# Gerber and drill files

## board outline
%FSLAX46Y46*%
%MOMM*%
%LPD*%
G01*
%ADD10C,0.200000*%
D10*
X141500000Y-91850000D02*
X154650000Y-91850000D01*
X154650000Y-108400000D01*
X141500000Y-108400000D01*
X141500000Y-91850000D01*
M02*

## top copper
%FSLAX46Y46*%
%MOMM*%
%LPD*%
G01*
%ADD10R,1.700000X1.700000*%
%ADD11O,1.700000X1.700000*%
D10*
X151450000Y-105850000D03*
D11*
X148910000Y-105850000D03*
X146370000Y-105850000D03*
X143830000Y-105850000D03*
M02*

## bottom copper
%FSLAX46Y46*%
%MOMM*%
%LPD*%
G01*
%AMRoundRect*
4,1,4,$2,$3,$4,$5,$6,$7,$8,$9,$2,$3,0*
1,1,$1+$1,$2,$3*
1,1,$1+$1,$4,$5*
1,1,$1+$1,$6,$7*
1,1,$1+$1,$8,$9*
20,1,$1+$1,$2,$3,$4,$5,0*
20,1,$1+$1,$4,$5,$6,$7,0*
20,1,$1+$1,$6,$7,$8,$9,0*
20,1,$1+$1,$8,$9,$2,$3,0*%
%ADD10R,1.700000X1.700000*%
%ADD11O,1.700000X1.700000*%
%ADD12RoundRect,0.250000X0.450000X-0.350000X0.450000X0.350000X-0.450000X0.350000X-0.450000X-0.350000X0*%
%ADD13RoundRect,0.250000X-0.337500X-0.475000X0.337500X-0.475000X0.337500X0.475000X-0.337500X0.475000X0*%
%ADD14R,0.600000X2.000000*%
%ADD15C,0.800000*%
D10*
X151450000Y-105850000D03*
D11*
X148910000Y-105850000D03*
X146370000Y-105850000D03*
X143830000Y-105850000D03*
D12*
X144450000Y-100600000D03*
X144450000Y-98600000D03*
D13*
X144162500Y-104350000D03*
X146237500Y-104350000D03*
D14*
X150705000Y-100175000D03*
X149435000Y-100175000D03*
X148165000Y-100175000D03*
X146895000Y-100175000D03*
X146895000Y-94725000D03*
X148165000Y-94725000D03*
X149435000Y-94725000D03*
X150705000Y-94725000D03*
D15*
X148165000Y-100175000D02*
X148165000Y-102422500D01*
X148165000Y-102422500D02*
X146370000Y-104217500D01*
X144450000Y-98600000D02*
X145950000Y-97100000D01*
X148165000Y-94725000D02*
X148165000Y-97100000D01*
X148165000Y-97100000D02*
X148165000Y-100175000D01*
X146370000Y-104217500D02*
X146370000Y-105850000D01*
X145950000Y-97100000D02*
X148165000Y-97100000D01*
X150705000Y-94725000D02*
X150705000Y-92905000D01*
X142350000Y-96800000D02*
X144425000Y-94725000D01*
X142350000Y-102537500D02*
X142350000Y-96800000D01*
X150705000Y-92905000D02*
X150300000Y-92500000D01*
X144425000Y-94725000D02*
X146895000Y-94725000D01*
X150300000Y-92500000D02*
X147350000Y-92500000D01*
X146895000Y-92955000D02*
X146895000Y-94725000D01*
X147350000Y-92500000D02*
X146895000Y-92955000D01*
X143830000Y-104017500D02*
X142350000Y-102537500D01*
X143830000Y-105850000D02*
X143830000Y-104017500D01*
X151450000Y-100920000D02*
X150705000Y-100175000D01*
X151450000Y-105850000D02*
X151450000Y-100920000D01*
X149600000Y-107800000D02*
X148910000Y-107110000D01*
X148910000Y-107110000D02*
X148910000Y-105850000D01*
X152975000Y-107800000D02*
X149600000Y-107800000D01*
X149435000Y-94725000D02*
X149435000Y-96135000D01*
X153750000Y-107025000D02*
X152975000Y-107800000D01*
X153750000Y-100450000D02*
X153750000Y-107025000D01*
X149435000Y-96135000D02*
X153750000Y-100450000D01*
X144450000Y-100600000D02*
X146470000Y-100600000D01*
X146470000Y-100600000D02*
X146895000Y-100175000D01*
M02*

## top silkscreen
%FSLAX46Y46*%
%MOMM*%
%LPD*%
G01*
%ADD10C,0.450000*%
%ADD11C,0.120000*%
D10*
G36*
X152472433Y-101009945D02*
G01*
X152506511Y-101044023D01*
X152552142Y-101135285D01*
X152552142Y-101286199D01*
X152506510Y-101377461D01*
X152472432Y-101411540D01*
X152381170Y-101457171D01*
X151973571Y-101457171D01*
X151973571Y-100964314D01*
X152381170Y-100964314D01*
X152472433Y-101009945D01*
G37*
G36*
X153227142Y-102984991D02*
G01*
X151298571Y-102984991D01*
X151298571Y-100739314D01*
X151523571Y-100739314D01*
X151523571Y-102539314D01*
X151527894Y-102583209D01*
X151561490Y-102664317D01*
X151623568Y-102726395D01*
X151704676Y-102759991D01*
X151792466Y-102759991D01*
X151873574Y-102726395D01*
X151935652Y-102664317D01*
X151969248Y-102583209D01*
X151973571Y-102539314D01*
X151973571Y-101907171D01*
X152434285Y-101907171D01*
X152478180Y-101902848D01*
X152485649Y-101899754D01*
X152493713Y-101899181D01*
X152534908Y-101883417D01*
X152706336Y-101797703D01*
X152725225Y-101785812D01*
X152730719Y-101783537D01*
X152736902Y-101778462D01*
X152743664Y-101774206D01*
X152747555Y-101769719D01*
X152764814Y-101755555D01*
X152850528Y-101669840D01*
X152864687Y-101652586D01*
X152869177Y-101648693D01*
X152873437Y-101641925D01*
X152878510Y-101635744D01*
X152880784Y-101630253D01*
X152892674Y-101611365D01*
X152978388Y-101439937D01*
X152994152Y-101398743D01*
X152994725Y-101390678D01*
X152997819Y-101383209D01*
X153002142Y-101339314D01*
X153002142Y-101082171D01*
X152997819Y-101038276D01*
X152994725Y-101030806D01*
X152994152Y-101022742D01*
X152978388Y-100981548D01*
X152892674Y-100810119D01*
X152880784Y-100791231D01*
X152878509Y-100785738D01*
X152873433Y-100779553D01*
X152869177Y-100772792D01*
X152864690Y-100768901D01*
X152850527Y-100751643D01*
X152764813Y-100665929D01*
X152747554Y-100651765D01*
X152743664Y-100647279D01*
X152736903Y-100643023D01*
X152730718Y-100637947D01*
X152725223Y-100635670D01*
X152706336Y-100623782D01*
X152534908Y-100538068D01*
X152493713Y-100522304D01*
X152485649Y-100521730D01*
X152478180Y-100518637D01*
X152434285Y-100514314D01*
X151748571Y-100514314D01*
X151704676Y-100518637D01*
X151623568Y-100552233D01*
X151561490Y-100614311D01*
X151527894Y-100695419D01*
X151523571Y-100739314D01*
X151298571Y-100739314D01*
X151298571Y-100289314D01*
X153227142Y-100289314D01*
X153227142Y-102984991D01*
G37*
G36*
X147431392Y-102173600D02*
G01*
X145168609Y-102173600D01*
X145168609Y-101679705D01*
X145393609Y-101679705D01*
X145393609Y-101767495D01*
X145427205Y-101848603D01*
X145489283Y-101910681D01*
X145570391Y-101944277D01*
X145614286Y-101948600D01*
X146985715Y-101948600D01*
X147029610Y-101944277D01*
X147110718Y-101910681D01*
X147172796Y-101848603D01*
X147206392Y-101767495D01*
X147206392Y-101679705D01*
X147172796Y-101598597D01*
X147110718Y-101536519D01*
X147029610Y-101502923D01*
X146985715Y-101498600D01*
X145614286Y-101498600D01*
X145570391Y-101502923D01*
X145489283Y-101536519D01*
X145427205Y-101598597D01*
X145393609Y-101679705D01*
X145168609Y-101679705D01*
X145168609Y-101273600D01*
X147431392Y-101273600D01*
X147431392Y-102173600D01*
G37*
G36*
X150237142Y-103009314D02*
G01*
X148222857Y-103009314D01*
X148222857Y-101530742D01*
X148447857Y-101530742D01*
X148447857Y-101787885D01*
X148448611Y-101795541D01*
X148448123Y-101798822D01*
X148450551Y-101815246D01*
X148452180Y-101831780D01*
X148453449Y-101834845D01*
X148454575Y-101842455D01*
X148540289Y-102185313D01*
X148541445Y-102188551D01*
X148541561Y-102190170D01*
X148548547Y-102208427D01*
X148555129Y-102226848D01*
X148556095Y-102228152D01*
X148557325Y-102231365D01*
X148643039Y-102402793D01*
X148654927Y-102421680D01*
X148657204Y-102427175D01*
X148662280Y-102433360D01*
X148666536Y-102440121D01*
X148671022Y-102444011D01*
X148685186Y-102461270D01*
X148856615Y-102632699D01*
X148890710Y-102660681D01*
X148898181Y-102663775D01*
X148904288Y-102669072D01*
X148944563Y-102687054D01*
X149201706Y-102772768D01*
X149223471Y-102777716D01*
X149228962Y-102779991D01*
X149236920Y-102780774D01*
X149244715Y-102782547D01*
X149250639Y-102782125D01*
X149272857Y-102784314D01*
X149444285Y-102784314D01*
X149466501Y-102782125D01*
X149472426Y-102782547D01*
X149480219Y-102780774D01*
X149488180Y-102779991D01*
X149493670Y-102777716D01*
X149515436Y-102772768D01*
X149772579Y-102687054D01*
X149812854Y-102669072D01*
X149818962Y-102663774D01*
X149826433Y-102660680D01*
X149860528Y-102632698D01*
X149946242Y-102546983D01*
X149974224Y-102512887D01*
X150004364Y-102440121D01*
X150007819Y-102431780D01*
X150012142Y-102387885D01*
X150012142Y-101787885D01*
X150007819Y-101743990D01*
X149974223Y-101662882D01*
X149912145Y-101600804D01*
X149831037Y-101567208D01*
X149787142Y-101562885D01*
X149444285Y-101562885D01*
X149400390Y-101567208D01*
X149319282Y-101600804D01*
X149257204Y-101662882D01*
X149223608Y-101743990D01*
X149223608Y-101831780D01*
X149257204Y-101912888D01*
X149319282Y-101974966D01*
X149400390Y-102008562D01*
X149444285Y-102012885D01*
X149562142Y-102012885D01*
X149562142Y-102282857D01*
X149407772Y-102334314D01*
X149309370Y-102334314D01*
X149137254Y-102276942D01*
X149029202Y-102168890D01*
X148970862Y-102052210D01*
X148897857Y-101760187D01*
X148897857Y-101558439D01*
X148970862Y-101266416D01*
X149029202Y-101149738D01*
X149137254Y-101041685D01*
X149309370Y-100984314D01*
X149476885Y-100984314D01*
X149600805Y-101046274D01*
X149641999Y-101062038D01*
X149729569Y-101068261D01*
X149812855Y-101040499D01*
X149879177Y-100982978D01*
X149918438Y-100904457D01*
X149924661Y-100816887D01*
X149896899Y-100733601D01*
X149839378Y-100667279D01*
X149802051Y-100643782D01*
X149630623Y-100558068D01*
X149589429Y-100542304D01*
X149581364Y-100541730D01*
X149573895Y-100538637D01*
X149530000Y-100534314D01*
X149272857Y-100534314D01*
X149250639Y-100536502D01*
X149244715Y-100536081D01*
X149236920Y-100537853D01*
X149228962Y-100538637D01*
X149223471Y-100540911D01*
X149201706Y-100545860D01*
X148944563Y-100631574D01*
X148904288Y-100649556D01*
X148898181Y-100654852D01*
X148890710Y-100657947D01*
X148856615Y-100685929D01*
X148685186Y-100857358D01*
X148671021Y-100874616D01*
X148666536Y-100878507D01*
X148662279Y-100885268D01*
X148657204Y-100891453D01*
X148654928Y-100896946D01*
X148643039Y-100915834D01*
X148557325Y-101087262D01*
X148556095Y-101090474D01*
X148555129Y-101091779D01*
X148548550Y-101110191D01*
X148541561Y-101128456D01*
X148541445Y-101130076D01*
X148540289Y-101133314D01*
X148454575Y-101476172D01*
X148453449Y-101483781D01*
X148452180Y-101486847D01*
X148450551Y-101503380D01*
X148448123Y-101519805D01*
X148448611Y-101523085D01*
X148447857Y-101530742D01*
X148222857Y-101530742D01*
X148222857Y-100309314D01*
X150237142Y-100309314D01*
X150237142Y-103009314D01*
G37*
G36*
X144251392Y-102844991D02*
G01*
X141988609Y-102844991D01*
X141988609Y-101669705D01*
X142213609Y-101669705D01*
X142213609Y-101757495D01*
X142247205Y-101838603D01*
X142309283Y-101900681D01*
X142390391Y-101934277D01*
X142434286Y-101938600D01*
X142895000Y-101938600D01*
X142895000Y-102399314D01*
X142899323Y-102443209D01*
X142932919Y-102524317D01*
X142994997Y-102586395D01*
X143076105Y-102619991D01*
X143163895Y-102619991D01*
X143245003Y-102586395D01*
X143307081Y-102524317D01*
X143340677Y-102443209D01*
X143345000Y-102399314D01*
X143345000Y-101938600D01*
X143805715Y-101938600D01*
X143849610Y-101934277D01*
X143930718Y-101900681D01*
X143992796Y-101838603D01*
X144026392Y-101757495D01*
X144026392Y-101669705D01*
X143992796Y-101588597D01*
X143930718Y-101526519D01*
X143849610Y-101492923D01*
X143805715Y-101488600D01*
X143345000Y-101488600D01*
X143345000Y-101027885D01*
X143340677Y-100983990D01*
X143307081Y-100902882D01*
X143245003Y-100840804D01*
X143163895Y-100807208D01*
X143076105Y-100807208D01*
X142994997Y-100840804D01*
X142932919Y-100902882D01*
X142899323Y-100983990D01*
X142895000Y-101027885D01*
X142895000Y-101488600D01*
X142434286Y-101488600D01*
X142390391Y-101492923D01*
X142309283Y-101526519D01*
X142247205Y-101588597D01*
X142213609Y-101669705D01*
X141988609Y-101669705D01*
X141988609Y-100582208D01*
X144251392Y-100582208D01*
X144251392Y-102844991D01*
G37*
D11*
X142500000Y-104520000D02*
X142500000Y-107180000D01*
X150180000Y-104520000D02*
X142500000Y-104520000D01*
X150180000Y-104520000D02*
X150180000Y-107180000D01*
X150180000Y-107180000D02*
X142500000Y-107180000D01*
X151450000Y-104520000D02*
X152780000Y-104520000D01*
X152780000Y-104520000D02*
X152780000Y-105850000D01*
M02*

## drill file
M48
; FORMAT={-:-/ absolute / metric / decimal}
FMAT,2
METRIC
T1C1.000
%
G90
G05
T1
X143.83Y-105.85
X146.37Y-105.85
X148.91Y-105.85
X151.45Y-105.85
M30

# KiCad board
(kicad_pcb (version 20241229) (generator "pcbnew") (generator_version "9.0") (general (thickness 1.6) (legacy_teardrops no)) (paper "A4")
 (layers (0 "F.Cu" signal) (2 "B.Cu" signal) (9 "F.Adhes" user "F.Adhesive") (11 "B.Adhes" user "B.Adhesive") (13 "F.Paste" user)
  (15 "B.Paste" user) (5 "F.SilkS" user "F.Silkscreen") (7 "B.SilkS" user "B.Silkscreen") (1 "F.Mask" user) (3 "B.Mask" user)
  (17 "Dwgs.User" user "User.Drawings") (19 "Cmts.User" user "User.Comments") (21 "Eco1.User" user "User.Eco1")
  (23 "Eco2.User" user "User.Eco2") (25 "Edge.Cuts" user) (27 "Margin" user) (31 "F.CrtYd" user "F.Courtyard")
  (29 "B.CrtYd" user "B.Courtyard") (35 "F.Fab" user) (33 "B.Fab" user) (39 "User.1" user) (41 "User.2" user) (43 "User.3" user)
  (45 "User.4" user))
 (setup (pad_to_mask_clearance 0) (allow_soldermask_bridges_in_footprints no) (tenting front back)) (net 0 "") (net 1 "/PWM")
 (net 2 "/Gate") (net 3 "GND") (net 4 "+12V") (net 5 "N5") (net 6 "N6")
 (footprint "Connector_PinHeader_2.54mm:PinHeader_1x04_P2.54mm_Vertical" (layer "F.Cu") (at 151.45 105.85 -90)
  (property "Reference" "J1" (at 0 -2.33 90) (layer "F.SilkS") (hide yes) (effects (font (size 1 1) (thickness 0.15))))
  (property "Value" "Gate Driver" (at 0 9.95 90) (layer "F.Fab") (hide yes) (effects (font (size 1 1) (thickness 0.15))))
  (fp_line (start -1.33 8.95) (end 1.33 8.95) (stroke (width 0.12) (type solid)) (layer "F.SilkS"))
  (fp_line (start -1.33 1.27) (end -1.33 8.95) (stroke (width 0.12) (type solid)) (layer "F.SilkS"))
  (fp_line (start -1.33 1.27) (end 1.33 1.27) (stroke (width 0.12) (type solid)) (layer "F.SilkS"))
  (fp_line (start 1.33 1.27) (end 1.33 8.95) (stroke (width 0.12) (type solid)) (layer "F.SilkS"))
  (fp_line (start -1.33 0) (end -1.33 -1.33) (stroke (width 0.12) (type solid)) (layer "F.SilkS"))
  (fp_line (start -1.33 -1.33) (end 0 -1.33) (stroke (width 0.12) (type solid)) (layer "F.SilkS"))
  (pad "1" thru_hole rect (at 0 0 270) (size 1.7 1.7) (drill 1) (layers "*.Cu" "*.Mask") (remove_unused_layers no) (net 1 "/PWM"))
  (pad "2" thru_hole oval (at 0 2.54 270) (size 1.7 1.7) (drill 1) (layers "*.Cu" "*.Mask") (remove_unused_layers no) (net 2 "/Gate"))
  (pad "3" thru_hole oval (at 0 5.08 270) (size 1.7 1.7) (drill 1) (layers "*.Cu" "*.Mask") (remove_unused_layers no) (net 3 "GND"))
  (pad "4" thru_hole oval (at 0 7.62 270) (size 1.7 1.7) (drill 1) (layers "*.Cu" "*.Mask") (remove_unused_layers no) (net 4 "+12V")))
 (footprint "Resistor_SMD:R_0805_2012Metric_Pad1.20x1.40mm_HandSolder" (layer "B.Cu") (at 144.45 99.6 90)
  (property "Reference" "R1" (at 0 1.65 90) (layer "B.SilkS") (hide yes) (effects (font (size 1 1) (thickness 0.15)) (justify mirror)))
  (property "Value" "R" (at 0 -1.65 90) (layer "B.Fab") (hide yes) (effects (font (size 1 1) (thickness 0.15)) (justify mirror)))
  (pad "1" smd roundrect (at -1 0 90) (size 1.2 1.4) (layers "B.Cu" "B.Mask" "B.Paste") (roundrect_rratio 0.208333) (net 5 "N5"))
  (pad "2" smd roundrect (at 1 0 90) (size 1.2 1.4) (layers "B.Cu" "B.Mask" "B.Paste") (roundrect_rratio 0.208333) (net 3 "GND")))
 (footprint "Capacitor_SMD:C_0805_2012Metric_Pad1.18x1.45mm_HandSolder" (layer "B.Cu") (at 145.2 104.35)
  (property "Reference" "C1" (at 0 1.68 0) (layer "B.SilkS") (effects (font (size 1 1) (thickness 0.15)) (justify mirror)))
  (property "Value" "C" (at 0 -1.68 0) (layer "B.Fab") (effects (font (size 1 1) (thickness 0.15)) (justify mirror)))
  (pad "1" smd roundrect (at -1.0375 0) (size 1.175 1.45) (layers "B.Cu" "B.Mask" "B.Paste") (roundrect_rratio 0.212766) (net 4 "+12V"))
  (pad "2" smd roundrect (at 1.0375 0) (size 1.175 1.45) (layers "B.Cu" "B.Mask" "B.Paste") (roundrect_rratio 0.212766) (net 3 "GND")))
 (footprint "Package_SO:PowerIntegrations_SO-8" (layer "B.Cu") (at 148.8 97.45 90)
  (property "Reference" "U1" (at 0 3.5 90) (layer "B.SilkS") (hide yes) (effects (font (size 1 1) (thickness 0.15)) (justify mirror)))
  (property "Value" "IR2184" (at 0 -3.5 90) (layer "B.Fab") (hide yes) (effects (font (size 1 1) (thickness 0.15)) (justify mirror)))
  (pad "1" smd rect (at -2.725 1.905 90) (size 2 0.6) (layers "B.Cu" "B.Mask" "B.Paste") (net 1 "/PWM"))
  (pad "2" smd rect (at -2.725 0.635 90) (size 2 0.6) (layers "B.Cu" "B.Mask" "B.Paste") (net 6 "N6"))
  (pad "3" smd rect (at -2.725 -0.635 90) (size 2 0.6) (layers "B.Cu" "B.Mask" "B.Paste") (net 3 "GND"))
  (pad "4" smd rect (at -2.725 -1.905 90) (size 2 0.6) (layers "B.Cu" "B.Mask" "B.Paste") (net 5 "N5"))
  (pad "5" smd rect (at 2.725 -1.905 90) (size 2 0.6) (layers "B.Cu" "B.Mask" "B.Paste") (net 4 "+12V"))
  (pad "6" smd rect (at 2.725 -0.635 90) (size 2 0.6) (layers "B.Cu" "B.Mask" "B.Paste") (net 3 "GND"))
  (pad "7" smd rect (at 2.725 0.635 90) (size 2 0.6) (layers "B.Cu" "B.Mask" "B.Paste") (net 2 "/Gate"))
  (pad "8" smd rect (at 2.725 1.905 90) (size 2 0.6) (layers "B.Cu" "B.Mask" "B.Paste") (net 4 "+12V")))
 (gr_rect (start 141.5 91.85) (end 154.65 108.4) (stroke (width 0.2) (type solid)) (fill no) (layer "Edge.Cuts"))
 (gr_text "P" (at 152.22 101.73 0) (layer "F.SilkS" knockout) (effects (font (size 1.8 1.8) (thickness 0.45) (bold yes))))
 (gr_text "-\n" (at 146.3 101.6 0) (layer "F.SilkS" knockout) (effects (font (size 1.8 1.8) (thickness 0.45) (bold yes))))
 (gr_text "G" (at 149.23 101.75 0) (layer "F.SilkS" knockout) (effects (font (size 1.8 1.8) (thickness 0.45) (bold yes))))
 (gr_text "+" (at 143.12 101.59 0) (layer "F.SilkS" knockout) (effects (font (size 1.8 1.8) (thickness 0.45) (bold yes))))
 (segment (start 148.165 100.175) (end 148.165 102.4225) (width 0.8) (layer "B.Cu") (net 3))
 (segment (start 148.165 102.4225) (end 146.37 104.2175) (width 0.8) (layer "B.Cu") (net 3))
 (segment (start 144.45 98.6) (end 145.95 97.1) (width 0.8) (layer "B.Cu") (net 3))
 (segment (start 148.165 94.725) (end 148.165 97.1) (width 0.8) (layer "B.Cu") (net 3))
 (segment (start 148.165 97.1) (end 148.165 100.175) (width 0.8) (layer "B.Cu") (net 3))
 (segment (start 146.37 104.2175) (end 146.37 105.85) (width 0.8) (layer "B.Cu") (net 3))
 (segment (start 145.95 97.1) (end 148.165 97.1) (width 0.8) (layer "B.Cu") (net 3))
 (segment (start 150.705 94.725) (end 150.705 92.905) (width 0.8) (layer "B.Cu") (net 4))
 (segment (start 142.35 96.8) (end 144.425 94.725) (width 0.8) (layer "B.Cu") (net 4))
 (segment (start 142.35 102.5375) (end 142.35 96.8) (width 0.8) (layer "B.Cu") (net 4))
 (segment (start 150.705 92.905) (end 150.3 92.5) (width 0.8) (layer "B.Cu") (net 4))
 (segment (start 144.425 94.725) (end 146.895 94.725) (width 0.8) (layer "B.Cu") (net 4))
 (segment (start 150.3 92.5) (end 147.35 92.5) (width 0.8) (layer "B.Cu") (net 4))
 (segment (start 146.895 92.955) (end 146.895 94.725) (width 0.8) (layer "B.Cu") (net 4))
 (segment (start 147.35 92.5) (end 146.895 92.955) (width 0.8) (layer "B.Cu") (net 4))
 (segment (start 143.83 104.0175) (end 142.35 102.5375) (width 0.8) (layer "B.Cu") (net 4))
 (segment (start 143.83 105.85) (end 143.83 104.0175) (width 0.8) (layer "B.Cu") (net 4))
 (segment (start 151.45 100.92) (end 150.705 100.175) (width 0.8) (layer "B.Cu") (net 1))
 (segment (start 151.45 105.85) (end 151.45 100.92) (width 0.8) (layer "B.Cu") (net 1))
 (segment (start 149.6 107.8) (end 148.91 107.11) (width 0.8) (layer "B.Cu") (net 2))
 (segment (start 148.91 107.11) (end 148.91 105.85) (width 0.8) (layer "B.Cu") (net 2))
 (segment (start 152.975 107.8) (end 149.6 107.8) (width 0.8) (layer "B.Cu") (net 2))
 (segment (start 149.435 94.725) (end 149.435 96.135) (width 0.8) (layer "B.Cu") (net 2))
 (segment (start 153.75 107.025) (end 152.975 107.8) (width 0.8) (layer "B.Cu") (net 2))
 (segment (start 153.75 100.45) (end 153.75 107.025) (width 0.8) (layer "B.Cu") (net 2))
 (segment (start 149.435 96.135) (end 153.75 100.45) (width 0.8) (layer "B.Cu") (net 2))
 (segment (start 144.45 100.6) (end 146.47 100.6) (width 0.8) (layer "B.Cu") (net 5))
 (segment (start 146.47 100.6) (end 146.895 100.175) (width 0.8) (layer "B.Cu") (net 5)))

